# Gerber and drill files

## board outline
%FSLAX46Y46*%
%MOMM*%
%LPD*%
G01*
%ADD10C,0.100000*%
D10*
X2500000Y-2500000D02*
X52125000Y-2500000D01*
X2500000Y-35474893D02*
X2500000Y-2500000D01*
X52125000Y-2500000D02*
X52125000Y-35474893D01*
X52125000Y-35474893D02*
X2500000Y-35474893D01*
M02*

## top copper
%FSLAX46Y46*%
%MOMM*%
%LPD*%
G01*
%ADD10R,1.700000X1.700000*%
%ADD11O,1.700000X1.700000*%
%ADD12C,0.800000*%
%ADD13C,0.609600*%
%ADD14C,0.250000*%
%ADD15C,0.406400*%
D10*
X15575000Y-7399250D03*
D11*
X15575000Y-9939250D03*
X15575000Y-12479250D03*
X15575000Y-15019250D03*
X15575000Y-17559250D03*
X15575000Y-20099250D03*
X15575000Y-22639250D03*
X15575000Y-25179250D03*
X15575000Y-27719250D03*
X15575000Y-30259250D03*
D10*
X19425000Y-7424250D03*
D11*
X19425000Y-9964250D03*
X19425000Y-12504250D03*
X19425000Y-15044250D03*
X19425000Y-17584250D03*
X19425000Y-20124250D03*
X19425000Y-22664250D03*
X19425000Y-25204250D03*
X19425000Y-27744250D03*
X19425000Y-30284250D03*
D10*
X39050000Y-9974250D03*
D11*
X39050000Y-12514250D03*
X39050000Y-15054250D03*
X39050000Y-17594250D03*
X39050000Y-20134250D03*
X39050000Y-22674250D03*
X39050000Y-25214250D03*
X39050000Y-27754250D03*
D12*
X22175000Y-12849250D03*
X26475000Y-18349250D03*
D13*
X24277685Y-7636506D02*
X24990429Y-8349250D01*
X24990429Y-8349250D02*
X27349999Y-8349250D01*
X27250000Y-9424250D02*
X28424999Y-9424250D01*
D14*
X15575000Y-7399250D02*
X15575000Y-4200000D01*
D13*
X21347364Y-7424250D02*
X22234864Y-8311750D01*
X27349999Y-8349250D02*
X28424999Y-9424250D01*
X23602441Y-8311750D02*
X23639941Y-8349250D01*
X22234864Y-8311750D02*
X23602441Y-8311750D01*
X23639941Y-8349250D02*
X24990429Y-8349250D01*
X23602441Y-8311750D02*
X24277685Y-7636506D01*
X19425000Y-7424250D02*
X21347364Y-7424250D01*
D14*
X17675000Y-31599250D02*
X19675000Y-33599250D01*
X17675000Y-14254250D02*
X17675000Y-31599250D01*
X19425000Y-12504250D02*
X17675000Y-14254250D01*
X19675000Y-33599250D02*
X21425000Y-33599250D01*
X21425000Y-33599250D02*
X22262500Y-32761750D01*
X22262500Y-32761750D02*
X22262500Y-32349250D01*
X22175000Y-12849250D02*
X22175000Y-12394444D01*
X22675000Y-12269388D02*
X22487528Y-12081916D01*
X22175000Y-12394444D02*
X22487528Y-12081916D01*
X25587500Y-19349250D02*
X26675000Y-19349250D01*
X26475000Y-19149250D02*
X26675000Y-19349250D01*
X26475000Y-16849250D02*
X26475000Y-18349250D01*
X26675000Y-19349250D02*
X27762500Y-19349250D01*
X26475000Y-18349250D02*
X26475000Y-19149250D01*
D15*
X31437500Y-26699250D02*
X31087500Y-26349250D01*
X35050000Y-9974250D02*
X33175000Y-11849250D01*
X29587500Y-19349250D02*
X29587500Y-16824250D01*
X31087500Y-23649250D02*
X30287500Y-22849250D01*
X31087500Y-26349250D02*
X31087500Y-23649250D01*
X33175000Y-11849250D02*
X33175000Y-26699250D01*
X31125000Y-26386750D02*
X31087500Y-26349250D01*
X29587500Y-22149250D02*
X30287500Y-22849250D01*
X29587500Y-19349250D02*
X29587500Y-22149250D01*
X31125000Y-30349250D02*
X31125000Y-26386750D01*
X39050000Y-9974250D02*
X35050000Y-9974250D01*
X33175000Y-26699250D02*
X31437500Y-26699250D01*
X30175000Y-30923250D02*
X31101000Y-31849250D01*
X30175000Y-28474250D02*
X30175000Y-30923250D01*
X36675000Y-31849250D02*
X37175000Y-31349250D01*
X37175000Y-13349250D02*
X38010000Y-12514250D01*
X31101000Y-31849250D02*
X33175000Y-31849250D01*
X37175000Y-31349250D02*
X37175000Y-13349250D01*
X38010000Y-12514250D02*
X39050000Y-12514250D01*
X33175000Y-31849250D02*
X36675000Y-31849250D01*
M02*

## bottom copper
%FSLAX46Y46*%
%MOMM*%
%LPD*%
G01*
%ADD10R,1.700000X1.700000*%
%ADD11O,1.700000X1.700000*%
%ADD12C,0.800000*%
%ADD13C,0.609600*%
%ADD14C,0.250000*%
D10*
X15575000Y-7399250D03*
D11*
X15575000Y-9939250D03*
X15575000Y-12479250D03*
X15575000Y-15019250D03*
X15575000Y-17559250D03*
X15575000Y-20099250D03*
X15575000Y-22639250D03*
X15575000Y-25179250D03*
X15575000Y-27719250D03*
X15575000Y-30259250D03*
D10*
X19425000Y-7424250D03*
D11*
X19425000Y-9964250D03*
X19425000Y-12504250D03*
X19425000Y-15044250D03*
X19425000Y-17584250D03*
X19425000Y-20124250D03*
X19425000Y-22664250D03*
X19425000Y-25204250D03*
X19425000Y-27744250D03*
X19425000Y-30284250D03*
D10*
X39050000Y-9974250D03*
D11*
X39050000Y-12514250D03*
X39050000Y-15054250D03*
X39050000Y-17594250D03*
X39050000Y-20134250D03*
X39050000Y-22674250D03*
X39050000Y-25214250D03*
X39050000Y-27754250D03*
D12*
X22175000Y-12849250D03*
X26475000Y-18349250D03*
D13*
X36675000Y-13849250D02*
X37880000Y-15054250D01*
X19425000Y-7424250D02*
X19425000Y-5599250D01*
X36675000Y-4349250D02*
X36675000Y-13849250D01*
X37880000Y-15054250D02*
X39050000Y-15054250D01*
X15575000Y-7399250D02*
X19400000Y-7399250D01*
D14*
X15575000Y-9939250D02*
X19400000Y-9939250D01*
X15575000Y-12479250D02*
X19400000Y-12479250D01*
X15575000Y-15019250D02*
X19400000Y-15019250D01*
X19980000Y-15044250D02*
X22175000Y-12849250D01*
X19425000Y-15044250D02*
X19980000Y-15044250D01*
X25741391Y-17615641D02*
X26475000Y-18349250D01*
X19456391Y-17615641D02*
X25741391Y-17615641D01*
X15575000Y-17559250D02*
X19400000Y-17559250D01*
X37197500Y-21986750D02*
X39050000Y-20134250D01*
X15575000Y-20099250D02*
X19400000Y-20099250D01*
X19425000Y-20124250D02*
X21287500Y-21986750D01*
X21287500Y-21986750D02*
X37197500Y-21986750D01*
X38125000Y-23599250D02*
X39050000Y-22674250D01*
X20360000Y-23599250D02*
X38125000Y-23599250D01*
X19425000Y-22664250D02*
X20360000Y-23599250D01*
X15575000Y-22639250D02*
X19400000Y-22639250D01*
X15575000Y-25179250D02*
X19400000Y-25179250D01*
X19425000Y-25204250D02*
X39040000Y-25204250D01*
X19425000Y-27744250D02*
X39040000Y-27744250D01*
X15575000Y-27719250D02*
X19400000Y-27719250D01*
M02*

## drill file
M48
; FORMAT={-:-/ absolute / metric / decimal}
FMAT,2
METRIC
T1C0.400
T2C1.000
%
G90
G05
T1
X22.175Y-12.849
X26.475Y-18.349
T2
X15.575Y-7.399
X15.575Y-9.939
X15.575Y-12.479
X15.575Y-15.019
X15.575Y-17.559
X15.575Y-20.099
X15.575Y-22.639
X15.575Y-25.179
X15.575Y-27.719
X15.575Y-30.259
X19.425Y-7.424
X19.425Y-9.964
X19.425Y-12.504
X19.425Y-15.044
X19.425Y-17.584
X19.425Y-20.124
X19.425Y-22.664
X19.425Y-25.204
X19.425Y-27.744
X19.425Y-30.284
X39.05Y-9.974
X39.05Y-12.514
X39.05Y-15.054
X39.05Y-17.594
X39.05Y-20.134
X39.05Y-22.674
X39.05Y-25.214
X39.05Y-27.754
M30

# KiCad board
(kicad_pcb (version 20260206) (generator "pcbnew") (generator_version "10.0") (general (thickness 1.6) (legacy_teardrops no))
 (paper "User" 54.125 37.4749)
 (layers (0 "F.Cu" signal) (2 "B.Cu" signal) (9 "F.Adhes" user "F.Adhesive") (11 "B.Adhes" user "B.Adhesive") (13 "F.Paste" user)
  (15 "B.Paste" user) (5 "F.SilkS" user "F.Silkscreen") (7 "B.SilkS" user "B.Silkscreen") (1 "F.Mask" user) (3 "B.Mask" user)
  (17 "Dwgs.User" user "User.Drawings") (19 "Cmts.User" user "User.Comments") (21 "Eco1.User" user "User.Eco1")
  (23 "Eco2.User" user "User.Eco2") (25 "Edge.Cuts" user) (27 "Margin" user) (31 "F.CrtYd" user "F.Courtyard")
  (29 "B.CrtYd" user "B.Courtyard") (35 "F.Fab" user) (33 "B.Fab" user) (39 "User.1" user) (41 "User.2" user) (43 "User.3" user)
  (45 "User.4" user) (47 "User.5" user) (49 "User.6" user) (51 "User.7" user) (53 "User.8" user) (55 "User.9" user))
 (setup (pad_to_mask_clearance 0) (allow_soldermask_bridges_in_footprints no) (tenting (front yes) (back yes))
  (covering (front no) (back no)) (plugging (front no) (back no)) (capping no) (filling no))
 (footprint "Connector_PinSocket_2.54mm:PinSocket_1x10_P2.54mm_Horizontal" (layer "F.Cu") (at 15.575 7.39925)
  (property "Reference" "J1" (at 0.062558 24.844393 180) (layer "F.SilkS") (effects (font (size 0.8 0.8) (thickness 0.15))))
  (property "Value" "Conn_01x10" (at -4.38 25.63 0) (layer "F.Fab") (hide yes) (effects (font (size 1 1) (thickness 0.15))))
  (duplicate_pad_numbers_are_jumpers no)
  (pad "1" thru_hole rect (at 0 0) (size 1.7 1.7) (drill 1) (layers "*.Cu" "*.Mask") (remove_unused_layers no) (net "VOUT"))
  (pad "2" thru_hole oval (at 0 2.54) (size 1.7 1.7) (drill 1) (layers "*.Cu" "*.Mask") (remove_unused_layers no) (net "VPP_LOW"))
  (pad "3" thru_hole oval (at 0 5.08) (size 1.7 1.7) (drill 1) (layers "*.Cu" "*.Mask") (remove_unused_layers no) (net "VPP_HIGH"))
  (pad "4" thru_hole oval (at 0 7.62) (size 1.7 1.7) (drill 1) (layers "*.Cu" "*.Mask") (remove_unused_layers no) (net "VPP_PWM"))
  (pad "5" thru_hole oval (at 0 10.16) (size 1.7 1.7) (drill 1) (layers "*.Cu" "*.Mask") (remove_unused_layers no) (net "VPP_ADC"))
  (pad "6" thru_hole oval (at 0 12.7) (size 1.7 1.7) (drill 1) (layers "*.Cu" "*.Mask") (remove_unused_layers no) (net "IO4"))
  (pad "7" thru_hole oval (at 0 15.24) (size 1.7 1.7) (drill 1) (layers "*.Cu" "*.Mask") (remove_unused_layers no) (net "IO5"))
  (pad "8" thru_hole oval (at 0 17.78) (size 1.7 1.7) (drill 1) (layers "*.Cu" "*.Mask") (remove_unused_layers no) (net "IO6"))
  (pad "9" thru_hole oval (at 0 20.32) (size 1.7 1.7) (drill 1) (layers "*.Cu" "*.Mask") (remove_unused_layers no) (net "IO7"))
  (pad "10" thru_hole oval (at 0 22.86) (size 1.7 1.7) (drill 1) (layers "*.Cu" "*.Mask") (remove_unused_layers no) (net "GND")))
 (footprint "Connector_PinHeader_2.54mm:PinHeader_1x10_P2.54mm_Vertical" (layer "F.Cu") (at 19.425 7.42425)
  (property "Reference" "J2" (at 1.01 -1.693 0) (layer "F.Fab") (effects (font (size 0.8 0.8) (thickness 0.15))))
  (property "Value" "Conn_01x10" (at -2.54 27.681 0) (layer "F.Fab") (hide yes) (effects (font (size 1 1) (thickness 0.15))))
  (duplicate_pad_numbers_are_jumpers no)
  (pad "1" thru_hole rect (at 0 0) (size 1.7 1.7) (drill 1) (layers "*.Cu" "*.Mask") (remove_unused_layers no) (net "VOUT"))
  (pad "2" thru_hole oval (at 0 2.54) (size 1.7 1.7) (drill 1) (layers "*.Cu" "*.Mask") (remove_unused_layers no) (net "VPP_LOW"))
  (pad "3" thru_hole oval (at 0 5.08) (size 1.7 1.7) (drill 1) (layers "*.Cu" "*.Mask") (remove_unused_layers no) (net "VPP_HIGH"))
  (pad "4" thru_hole oval (at 0 7.62) (size 1.7 1.7) (drill 1) (layers "*.Cu" "*.Mask") (remove_unused_layers no) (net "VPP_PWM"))
  (pad "5" thru_hole oval (at 0 10.16) (size 1.7 1.7) (drill 1) (layers "*.Cu" "*.Mask") (remove_unused_layers no) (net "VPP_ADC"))
  (pad "6" thru_hole oval (at 0 12.7) (size 1.7 1.7) (drill 1) (layers "*.Cu" "*.Mask") (remove_unused_layers no) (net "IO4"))
  (pad "7" thru_hole oval (at 0 15.24) (size 1.7 1.7) (drill 1) (layers "*.Cu" "*.Mask") (remove_unused_layers no) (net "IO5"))
  (pad "8" thru_hole oval (at 0 17.78) (size 1.7 1.7) (drill 1) (layers "*.Cu" "*.Mask") (remove_unused_layers no) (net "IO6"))
  (pad "9" thru_hole oval (at 0 20.32) (size 1.7 1.7) (drill 1) (layers "*.Cu" "*.Mask") (remove_unused_layers no) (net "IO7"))
  (pad "10" thru_hole oval (at 0 22.86) (size 1.7 1.7) (drill 1) (layers "*.Cu" "*.Mask") (remove_unused_layers no) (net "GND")))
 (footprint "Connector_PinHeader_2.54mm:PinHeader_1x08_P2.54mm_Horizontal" (layer "F.Cu") (at 39.05 9.97425)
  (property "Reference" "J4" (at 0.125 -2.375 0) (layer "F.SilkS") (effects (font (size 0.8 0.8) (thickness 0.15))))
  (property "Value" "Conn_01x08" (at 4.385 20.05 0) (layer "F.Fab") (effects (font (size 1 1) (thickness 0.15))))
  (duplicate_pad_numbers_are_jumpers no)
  (pad "1" thru_hole rect (at 0 0) (size 1.7 1.7) (drill 1) (layers "*.Cu" "*.Mask") (remove_unused_layers no) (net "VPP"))
  (pad "2" thru_hole oval (at 0 2.54) (size 1.7 1.7) (drill 1) (layers "*.Cu" "*.Mask") (remove_unused_layers no) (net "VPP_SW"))
  (pad "3" thru_hole oval (at 0 5.08) (size 1.7 1.7) (drill 1) (layers "*.Cu" "*.Mask") (remove_unused_layers no) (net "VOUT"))
  (pad "4" thru_hole oval (at 0 7.62) (size 1.7 1.7) (drill 1) (layers "*.Cu" "*.Mask") (remove_unused_layers no) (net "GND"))
  (pad "5" thru_hole oval (at 0 10.16) (size 1.7 1.7) (drill 1) (layers "*.Cu" "*.Mask") (remove_unused_layers no) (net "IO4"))
  (pad "6" thru_hole oval (at 0 12.7) (size 1.7 1.7) (drill 1) (layers "*.Cu" "*.Mask") (remove_unused_layers no) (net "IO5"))
  (pad "7" thru_hole oval (at 0 15.24) (size 1.7 1.7) (drill 1) (layers "*.Cu" "*.Mask") (remove_unused_layers no) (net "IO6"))
  (pad "8" thru_hole oval (at 0 17.78) (size 1.7 1.7) (drill 1) (layers "*.Cu" "*.Mask") (remove_unused_layers no) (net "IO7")))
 (gr_line (start 2.5 2.5) (end 52.125 2.5) (stroke (width 0.1) (type default)) (layer "Edge.Cuts"))
 (gr_line (start 2.5 35.474893) (end 2.5 2.5) (stroke (width 0.1) (type default)) (layer "Edge.Cuts"))
 (gr_line (start 52.125 2.5) (end 52.125 35.474893) (stroke (width 0.1) (type default)) (layer "Edge.Cuts"))
 (gr_line (start 52.125 35.474893) (end 2.5 35.474893) (stroke (width 0.1) (type default)) (layer "Edge.Cuts"))
 (segment (start 24.277685 7.636506) (end 24.990429 8.34925) (width 0.6096) (layer "F.Cu") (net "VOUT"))
 (segment (start 24.990429 8.34925) (end 27.349999 8.34925) (width 0.6096) (layer "F.Cu") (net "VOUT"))
 (segment (start 27.25 9.42425) (end 28.424999 9.42425) (width 0.6096) (layer "F.Cu") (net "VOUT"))
 (segment (start 15.575 7.39925) (end 15.575 4.2) (width 0.25) (layer "F.Cu") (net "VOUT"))
 (segment (start 21.347364 7.42425) (end 22.234864 8.31175) (width 0.6096) (layer "F.Cu") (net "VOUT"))
 (segment (start 27.349999 8.34925) (end 28.424999 9.42425) (width 0.6096) (layer "F.Cu") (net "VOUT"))
 (segment (start 23.602441 8.31175) (end 23.639941 8.34925) (width 0.6096) (layer "F.Cu") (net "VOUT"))
 (segment (start 22.234864 8.31175) (end 23.602441 8.31175) (width 0.6096) (layer "F.Cu") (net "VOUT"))
 (segment (start 23.639941 8.34925) (end 24.990429 8.34925) (width 0.6096) (layer "F.Cu") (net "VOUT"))
 (segment (start 23.602441 8.31175) (end 24.277685 7.636506) (width 0.6096) (layer "F.Cu") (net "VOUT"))
 (segment (start 19.425 7.42425) (end 21.347364 7.42425) (width 0.6096) (layer "F.Cu") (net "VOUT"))
 (segment (start 36.675 13.84925) (end 37.88 15.05425) (width 0.6096) (layer "B.Cu") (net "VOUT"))
 (segment (start 19.425 7.42425) (end 19.425 5.59925) (width 0.6096) (layer "B.Cu") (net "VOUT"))
 (segment (start 36.675 4.34925) (end 36.675 13.84925) (width 0.6096) (layer "B.Cu") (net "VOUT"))
 (segment (start 37.88 15.05425) (end 39.05 15.05425) (width 0.6096) (layer "B.Cu") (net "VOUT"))
 (segment (start 15.575 7.39925) (end 19.4 7.39925) (width 0.6096) (layer "B.Cu") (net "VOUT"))
 (segment (start 15.575 9.93925) (end 19.4 9.93925) (width 0.25) (layer "B.Cu") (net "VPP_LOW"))
 (segment (start 17.675 31.59925) (end 19.675 33.59925) (width 0.25) (layer "F.Cu") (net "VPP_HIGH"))
 (segment (start 17.675 14.25425) (end 17.675 31.59925) (width 0.25) (layer "F.Cu") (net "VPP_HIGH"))
 (segment (start 19.425 12.50425) (end 17.675 14.25425) (width 0.25) (layer "F.Cu") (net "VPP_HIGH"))
 (segment (start 19.675 33.59925) (end 21.425 33.59925) (width 0.25) (layer "F.Cu") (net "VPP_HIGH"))
 (segment (start 21.425 33.59925) (end 22.2625 32.76175) (width 0.25) (layer "F.Cu") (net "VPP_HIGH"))
 (segment (start 22.2625 32.76175) (end 22.2625 32.34925) (width 0.25) (layer "F.Cu") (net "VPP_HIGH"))
 (segment (start 15.575 12.47925) (end 19.4 12.47925) (width 0.25) (layer "B.Cu") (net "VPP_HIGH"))
 (segment (start 22.175 12.84925) (end 22.175 12.394444) (width 0.25) (layer "F.Cu") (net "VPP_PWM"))
 (segment (start 22.675 12.269388) (end 22.487528 12.081916) (width 0.25) (layer "F.Cu") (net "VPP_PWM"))
 (segment (start 22.175 12.394444) (end 22.487528 12.081916) (width 0.25) (layer "F.Cu") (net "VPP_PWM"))
 (via (at 22.175 12.84925) (size 0.8) (drill 0.4) (layers "F.Cu" "B.Cu") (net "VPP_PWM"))
 (segment (start 15.575 15.01925) (end 19.4 15.01925) (width 0.25) (layer "B.Cu") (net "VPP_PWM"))
 (segment (start 19.98 15.04425) (end 22.175 12.84925) (width 0.25) (layer "B.Cu") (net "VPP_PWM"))
 (segment (start 19.425 15.04425) (end 19.98 15.04425) (width 0.25) (layer "B.Cu") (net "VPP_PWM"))
 (segment (start 25.5875 19.34925) (end 26.675 19.34925) (width 0.25) (layer "F.Cu") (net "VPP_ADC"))
 (segment (start 26.475 19.14925) (end 26.675 19.34925) (width 0.25) (layer "F.Cu") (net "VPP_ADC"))
 (segment (start 26.475 16.84925) (end 26.475 18.34925) (width 0.25) (layer "F.Cu") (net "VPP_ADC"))
 (segment (start 26.675 19.34925) (end 27.7625 19.34925) (width 0.25) (layer "F.Cu") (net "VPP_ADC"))
 (segment (start 26.475 18.34925) (end 26.475 19.14925) (width 0.25) (layer "F.Cu") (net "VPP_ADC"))
 (via (at 26.475 18.34925) (size 0.8) (drill 0.4) (layers "F.Cu" "B.Cu") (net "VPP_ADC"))
 (segment (start 25.741391 17.615641) (end 26.475 18.34925) (width 0.25) (layer "B.Cu") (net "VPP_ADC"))
 (segment (start 19.456391 17.615641) (end 25.741391 17.615641) (width 0.25) (layer "B.Cu") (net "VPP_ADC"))
 (segment (start 15.575 17.55925) (end 19.4 17.55925) (width 0.25) (layer "B.Cu") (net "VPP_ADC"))
 (segment (start 37.1975 21.98675) (end 39.05 20.13425) (width 0.25) (layer "B.Cu") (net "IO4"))
 (segment (start 15.575 20.09925) (end 19.4 20.09925) (width 0.25) (layer "B.Cu") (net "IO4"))
 (segment (start 19.425 20.12425) (end 21.2875 21.98675) (width 0.25) (layer "B.Cu") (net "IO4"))
 (segment (start 21.2875 21.98675) (end 37.1975 21.98675) (width 0.25) (layer "B.Cu") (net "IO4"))
 (segment (start 38.125 23.59925) (end 39.05 22.67425) (width 0.25) (layer "B.Cu") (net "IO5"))
 (segment (start 20.36 23.59925) (end 38.125 23.59925) (width 0.25) (layer "B.Cu") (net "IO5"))
 (segment (start 19.425 22.66425) (end 20.36 23.59925) (width 0.25) (layer "B.Cu") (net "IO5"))
 (segment (start 15.575 22.63925) (end 19.4 22.63925) (width 0.25) (layer "B.Cu") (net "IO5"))
 (segment (start 15.575 25.17925) (end 19.4 25.17925) (width 0.25) (layer "B.Cu") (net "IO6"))
 (segment (start 19.425 25.20425) (end 39.04 25.20425) (width 0.25) (layer "B.Cu") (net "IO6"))
 (segment (start 19.425 27.74425) (end 39.04 27.74425) (width 0.25) (layer "B.Cu") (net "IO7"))
 (segment (start 15.575 27.71925) (end 19.4 27.71925) (width 0.25) (layer "B.Cu") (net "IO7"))
 (segment (start 31.4375 26.69925) (end 31.0875 26.34925) (width 0.4064) (layer "F.Cu") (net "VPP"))
 (segment (start 35.05 9.97425) (end 33.175 11.84925) (width 0.4064) (layer "F.Cu") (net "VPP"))
 (segment (start 29.5875 19.34925) (end 29.5875 16.82425) (width 0.4064) (layer "F.Cu") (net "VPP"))
 (segment (start 31.0875 23.64925) (end 30.2875 22.84925) (width 0.4064) (layer "F.Cu") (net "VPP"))
 (segment (start 31.0875 26.34925) (end 31.0875 23.64925) (width 0.4064) (layer "F.Cu") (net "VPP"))
 (segment (start 33.175 11.84925) (end 33.175 26.69925) (width 0.4064) (layer "F.Cu") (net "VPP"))
 (segment (start 31.125 26.38675) (end 31.0875 26.34925) (width 0.4064) (layer "F.Cu") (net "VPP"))
 (segment (start 29.5875 22.14925) (end 30.2875 22.84925) (width 0.4064) (layer "F.Cu") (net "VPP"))
 (segment (start 29.5875 19.34925) (end 29.5875 22.14925) (width 0.4064) (layer "F.Cu") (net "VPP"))
 (segment (start 31.125 30.34925) (end 31.125 26.38675) (width 0.4064) (layer "F.Cu") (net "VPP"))
 (segment (start 39.05 9.97425) (end 35.05 9.97425) (width 0.4064) (layer "F.Cu") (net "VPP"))
 (segment (start 33.175 26.69925) (end 31.4375 26.69925) (width 0.4064) (layer "F.Cu") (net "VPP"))
 (segment (start 30.175 30.92325) (end 31.101 31.84925) (width 0.4064) (layer "F.Cu") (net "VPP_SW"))
 (segment (start 30.175 28.47425) (end 30.175 30.92325) (width 0.4064) (layer "F.Cu") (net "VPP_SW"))
 (segment (start 36.675 31.84925) (end 37.175 31.34925) (width 0.4064) (layer "F.Cu") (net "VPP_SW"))
 (segment (start 37.175 13.34925) (end 38.01 12.51425) (width 0.4064) (layer "F.Cu") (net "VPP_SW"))
 (segment (start 31.101 31.84925) (end 33.175 31.84925) (width 0.4064) (layer "F.Cu") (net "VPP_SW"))
 (segment (start 37.175 31.34925) (end 37.175 13.34925) (width 0.4064) (layer "F.Cu") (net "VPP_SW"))
 (segment (start 38.01 12.51425) (end 39.05 12.51425) (width 0.4064) (layer "F.Cu") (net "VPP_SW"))
 (segment (start 33.175 31.84925) (end 36.675 31.84925) (width 0.4064) (layer "F.Cu") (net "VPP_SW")))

